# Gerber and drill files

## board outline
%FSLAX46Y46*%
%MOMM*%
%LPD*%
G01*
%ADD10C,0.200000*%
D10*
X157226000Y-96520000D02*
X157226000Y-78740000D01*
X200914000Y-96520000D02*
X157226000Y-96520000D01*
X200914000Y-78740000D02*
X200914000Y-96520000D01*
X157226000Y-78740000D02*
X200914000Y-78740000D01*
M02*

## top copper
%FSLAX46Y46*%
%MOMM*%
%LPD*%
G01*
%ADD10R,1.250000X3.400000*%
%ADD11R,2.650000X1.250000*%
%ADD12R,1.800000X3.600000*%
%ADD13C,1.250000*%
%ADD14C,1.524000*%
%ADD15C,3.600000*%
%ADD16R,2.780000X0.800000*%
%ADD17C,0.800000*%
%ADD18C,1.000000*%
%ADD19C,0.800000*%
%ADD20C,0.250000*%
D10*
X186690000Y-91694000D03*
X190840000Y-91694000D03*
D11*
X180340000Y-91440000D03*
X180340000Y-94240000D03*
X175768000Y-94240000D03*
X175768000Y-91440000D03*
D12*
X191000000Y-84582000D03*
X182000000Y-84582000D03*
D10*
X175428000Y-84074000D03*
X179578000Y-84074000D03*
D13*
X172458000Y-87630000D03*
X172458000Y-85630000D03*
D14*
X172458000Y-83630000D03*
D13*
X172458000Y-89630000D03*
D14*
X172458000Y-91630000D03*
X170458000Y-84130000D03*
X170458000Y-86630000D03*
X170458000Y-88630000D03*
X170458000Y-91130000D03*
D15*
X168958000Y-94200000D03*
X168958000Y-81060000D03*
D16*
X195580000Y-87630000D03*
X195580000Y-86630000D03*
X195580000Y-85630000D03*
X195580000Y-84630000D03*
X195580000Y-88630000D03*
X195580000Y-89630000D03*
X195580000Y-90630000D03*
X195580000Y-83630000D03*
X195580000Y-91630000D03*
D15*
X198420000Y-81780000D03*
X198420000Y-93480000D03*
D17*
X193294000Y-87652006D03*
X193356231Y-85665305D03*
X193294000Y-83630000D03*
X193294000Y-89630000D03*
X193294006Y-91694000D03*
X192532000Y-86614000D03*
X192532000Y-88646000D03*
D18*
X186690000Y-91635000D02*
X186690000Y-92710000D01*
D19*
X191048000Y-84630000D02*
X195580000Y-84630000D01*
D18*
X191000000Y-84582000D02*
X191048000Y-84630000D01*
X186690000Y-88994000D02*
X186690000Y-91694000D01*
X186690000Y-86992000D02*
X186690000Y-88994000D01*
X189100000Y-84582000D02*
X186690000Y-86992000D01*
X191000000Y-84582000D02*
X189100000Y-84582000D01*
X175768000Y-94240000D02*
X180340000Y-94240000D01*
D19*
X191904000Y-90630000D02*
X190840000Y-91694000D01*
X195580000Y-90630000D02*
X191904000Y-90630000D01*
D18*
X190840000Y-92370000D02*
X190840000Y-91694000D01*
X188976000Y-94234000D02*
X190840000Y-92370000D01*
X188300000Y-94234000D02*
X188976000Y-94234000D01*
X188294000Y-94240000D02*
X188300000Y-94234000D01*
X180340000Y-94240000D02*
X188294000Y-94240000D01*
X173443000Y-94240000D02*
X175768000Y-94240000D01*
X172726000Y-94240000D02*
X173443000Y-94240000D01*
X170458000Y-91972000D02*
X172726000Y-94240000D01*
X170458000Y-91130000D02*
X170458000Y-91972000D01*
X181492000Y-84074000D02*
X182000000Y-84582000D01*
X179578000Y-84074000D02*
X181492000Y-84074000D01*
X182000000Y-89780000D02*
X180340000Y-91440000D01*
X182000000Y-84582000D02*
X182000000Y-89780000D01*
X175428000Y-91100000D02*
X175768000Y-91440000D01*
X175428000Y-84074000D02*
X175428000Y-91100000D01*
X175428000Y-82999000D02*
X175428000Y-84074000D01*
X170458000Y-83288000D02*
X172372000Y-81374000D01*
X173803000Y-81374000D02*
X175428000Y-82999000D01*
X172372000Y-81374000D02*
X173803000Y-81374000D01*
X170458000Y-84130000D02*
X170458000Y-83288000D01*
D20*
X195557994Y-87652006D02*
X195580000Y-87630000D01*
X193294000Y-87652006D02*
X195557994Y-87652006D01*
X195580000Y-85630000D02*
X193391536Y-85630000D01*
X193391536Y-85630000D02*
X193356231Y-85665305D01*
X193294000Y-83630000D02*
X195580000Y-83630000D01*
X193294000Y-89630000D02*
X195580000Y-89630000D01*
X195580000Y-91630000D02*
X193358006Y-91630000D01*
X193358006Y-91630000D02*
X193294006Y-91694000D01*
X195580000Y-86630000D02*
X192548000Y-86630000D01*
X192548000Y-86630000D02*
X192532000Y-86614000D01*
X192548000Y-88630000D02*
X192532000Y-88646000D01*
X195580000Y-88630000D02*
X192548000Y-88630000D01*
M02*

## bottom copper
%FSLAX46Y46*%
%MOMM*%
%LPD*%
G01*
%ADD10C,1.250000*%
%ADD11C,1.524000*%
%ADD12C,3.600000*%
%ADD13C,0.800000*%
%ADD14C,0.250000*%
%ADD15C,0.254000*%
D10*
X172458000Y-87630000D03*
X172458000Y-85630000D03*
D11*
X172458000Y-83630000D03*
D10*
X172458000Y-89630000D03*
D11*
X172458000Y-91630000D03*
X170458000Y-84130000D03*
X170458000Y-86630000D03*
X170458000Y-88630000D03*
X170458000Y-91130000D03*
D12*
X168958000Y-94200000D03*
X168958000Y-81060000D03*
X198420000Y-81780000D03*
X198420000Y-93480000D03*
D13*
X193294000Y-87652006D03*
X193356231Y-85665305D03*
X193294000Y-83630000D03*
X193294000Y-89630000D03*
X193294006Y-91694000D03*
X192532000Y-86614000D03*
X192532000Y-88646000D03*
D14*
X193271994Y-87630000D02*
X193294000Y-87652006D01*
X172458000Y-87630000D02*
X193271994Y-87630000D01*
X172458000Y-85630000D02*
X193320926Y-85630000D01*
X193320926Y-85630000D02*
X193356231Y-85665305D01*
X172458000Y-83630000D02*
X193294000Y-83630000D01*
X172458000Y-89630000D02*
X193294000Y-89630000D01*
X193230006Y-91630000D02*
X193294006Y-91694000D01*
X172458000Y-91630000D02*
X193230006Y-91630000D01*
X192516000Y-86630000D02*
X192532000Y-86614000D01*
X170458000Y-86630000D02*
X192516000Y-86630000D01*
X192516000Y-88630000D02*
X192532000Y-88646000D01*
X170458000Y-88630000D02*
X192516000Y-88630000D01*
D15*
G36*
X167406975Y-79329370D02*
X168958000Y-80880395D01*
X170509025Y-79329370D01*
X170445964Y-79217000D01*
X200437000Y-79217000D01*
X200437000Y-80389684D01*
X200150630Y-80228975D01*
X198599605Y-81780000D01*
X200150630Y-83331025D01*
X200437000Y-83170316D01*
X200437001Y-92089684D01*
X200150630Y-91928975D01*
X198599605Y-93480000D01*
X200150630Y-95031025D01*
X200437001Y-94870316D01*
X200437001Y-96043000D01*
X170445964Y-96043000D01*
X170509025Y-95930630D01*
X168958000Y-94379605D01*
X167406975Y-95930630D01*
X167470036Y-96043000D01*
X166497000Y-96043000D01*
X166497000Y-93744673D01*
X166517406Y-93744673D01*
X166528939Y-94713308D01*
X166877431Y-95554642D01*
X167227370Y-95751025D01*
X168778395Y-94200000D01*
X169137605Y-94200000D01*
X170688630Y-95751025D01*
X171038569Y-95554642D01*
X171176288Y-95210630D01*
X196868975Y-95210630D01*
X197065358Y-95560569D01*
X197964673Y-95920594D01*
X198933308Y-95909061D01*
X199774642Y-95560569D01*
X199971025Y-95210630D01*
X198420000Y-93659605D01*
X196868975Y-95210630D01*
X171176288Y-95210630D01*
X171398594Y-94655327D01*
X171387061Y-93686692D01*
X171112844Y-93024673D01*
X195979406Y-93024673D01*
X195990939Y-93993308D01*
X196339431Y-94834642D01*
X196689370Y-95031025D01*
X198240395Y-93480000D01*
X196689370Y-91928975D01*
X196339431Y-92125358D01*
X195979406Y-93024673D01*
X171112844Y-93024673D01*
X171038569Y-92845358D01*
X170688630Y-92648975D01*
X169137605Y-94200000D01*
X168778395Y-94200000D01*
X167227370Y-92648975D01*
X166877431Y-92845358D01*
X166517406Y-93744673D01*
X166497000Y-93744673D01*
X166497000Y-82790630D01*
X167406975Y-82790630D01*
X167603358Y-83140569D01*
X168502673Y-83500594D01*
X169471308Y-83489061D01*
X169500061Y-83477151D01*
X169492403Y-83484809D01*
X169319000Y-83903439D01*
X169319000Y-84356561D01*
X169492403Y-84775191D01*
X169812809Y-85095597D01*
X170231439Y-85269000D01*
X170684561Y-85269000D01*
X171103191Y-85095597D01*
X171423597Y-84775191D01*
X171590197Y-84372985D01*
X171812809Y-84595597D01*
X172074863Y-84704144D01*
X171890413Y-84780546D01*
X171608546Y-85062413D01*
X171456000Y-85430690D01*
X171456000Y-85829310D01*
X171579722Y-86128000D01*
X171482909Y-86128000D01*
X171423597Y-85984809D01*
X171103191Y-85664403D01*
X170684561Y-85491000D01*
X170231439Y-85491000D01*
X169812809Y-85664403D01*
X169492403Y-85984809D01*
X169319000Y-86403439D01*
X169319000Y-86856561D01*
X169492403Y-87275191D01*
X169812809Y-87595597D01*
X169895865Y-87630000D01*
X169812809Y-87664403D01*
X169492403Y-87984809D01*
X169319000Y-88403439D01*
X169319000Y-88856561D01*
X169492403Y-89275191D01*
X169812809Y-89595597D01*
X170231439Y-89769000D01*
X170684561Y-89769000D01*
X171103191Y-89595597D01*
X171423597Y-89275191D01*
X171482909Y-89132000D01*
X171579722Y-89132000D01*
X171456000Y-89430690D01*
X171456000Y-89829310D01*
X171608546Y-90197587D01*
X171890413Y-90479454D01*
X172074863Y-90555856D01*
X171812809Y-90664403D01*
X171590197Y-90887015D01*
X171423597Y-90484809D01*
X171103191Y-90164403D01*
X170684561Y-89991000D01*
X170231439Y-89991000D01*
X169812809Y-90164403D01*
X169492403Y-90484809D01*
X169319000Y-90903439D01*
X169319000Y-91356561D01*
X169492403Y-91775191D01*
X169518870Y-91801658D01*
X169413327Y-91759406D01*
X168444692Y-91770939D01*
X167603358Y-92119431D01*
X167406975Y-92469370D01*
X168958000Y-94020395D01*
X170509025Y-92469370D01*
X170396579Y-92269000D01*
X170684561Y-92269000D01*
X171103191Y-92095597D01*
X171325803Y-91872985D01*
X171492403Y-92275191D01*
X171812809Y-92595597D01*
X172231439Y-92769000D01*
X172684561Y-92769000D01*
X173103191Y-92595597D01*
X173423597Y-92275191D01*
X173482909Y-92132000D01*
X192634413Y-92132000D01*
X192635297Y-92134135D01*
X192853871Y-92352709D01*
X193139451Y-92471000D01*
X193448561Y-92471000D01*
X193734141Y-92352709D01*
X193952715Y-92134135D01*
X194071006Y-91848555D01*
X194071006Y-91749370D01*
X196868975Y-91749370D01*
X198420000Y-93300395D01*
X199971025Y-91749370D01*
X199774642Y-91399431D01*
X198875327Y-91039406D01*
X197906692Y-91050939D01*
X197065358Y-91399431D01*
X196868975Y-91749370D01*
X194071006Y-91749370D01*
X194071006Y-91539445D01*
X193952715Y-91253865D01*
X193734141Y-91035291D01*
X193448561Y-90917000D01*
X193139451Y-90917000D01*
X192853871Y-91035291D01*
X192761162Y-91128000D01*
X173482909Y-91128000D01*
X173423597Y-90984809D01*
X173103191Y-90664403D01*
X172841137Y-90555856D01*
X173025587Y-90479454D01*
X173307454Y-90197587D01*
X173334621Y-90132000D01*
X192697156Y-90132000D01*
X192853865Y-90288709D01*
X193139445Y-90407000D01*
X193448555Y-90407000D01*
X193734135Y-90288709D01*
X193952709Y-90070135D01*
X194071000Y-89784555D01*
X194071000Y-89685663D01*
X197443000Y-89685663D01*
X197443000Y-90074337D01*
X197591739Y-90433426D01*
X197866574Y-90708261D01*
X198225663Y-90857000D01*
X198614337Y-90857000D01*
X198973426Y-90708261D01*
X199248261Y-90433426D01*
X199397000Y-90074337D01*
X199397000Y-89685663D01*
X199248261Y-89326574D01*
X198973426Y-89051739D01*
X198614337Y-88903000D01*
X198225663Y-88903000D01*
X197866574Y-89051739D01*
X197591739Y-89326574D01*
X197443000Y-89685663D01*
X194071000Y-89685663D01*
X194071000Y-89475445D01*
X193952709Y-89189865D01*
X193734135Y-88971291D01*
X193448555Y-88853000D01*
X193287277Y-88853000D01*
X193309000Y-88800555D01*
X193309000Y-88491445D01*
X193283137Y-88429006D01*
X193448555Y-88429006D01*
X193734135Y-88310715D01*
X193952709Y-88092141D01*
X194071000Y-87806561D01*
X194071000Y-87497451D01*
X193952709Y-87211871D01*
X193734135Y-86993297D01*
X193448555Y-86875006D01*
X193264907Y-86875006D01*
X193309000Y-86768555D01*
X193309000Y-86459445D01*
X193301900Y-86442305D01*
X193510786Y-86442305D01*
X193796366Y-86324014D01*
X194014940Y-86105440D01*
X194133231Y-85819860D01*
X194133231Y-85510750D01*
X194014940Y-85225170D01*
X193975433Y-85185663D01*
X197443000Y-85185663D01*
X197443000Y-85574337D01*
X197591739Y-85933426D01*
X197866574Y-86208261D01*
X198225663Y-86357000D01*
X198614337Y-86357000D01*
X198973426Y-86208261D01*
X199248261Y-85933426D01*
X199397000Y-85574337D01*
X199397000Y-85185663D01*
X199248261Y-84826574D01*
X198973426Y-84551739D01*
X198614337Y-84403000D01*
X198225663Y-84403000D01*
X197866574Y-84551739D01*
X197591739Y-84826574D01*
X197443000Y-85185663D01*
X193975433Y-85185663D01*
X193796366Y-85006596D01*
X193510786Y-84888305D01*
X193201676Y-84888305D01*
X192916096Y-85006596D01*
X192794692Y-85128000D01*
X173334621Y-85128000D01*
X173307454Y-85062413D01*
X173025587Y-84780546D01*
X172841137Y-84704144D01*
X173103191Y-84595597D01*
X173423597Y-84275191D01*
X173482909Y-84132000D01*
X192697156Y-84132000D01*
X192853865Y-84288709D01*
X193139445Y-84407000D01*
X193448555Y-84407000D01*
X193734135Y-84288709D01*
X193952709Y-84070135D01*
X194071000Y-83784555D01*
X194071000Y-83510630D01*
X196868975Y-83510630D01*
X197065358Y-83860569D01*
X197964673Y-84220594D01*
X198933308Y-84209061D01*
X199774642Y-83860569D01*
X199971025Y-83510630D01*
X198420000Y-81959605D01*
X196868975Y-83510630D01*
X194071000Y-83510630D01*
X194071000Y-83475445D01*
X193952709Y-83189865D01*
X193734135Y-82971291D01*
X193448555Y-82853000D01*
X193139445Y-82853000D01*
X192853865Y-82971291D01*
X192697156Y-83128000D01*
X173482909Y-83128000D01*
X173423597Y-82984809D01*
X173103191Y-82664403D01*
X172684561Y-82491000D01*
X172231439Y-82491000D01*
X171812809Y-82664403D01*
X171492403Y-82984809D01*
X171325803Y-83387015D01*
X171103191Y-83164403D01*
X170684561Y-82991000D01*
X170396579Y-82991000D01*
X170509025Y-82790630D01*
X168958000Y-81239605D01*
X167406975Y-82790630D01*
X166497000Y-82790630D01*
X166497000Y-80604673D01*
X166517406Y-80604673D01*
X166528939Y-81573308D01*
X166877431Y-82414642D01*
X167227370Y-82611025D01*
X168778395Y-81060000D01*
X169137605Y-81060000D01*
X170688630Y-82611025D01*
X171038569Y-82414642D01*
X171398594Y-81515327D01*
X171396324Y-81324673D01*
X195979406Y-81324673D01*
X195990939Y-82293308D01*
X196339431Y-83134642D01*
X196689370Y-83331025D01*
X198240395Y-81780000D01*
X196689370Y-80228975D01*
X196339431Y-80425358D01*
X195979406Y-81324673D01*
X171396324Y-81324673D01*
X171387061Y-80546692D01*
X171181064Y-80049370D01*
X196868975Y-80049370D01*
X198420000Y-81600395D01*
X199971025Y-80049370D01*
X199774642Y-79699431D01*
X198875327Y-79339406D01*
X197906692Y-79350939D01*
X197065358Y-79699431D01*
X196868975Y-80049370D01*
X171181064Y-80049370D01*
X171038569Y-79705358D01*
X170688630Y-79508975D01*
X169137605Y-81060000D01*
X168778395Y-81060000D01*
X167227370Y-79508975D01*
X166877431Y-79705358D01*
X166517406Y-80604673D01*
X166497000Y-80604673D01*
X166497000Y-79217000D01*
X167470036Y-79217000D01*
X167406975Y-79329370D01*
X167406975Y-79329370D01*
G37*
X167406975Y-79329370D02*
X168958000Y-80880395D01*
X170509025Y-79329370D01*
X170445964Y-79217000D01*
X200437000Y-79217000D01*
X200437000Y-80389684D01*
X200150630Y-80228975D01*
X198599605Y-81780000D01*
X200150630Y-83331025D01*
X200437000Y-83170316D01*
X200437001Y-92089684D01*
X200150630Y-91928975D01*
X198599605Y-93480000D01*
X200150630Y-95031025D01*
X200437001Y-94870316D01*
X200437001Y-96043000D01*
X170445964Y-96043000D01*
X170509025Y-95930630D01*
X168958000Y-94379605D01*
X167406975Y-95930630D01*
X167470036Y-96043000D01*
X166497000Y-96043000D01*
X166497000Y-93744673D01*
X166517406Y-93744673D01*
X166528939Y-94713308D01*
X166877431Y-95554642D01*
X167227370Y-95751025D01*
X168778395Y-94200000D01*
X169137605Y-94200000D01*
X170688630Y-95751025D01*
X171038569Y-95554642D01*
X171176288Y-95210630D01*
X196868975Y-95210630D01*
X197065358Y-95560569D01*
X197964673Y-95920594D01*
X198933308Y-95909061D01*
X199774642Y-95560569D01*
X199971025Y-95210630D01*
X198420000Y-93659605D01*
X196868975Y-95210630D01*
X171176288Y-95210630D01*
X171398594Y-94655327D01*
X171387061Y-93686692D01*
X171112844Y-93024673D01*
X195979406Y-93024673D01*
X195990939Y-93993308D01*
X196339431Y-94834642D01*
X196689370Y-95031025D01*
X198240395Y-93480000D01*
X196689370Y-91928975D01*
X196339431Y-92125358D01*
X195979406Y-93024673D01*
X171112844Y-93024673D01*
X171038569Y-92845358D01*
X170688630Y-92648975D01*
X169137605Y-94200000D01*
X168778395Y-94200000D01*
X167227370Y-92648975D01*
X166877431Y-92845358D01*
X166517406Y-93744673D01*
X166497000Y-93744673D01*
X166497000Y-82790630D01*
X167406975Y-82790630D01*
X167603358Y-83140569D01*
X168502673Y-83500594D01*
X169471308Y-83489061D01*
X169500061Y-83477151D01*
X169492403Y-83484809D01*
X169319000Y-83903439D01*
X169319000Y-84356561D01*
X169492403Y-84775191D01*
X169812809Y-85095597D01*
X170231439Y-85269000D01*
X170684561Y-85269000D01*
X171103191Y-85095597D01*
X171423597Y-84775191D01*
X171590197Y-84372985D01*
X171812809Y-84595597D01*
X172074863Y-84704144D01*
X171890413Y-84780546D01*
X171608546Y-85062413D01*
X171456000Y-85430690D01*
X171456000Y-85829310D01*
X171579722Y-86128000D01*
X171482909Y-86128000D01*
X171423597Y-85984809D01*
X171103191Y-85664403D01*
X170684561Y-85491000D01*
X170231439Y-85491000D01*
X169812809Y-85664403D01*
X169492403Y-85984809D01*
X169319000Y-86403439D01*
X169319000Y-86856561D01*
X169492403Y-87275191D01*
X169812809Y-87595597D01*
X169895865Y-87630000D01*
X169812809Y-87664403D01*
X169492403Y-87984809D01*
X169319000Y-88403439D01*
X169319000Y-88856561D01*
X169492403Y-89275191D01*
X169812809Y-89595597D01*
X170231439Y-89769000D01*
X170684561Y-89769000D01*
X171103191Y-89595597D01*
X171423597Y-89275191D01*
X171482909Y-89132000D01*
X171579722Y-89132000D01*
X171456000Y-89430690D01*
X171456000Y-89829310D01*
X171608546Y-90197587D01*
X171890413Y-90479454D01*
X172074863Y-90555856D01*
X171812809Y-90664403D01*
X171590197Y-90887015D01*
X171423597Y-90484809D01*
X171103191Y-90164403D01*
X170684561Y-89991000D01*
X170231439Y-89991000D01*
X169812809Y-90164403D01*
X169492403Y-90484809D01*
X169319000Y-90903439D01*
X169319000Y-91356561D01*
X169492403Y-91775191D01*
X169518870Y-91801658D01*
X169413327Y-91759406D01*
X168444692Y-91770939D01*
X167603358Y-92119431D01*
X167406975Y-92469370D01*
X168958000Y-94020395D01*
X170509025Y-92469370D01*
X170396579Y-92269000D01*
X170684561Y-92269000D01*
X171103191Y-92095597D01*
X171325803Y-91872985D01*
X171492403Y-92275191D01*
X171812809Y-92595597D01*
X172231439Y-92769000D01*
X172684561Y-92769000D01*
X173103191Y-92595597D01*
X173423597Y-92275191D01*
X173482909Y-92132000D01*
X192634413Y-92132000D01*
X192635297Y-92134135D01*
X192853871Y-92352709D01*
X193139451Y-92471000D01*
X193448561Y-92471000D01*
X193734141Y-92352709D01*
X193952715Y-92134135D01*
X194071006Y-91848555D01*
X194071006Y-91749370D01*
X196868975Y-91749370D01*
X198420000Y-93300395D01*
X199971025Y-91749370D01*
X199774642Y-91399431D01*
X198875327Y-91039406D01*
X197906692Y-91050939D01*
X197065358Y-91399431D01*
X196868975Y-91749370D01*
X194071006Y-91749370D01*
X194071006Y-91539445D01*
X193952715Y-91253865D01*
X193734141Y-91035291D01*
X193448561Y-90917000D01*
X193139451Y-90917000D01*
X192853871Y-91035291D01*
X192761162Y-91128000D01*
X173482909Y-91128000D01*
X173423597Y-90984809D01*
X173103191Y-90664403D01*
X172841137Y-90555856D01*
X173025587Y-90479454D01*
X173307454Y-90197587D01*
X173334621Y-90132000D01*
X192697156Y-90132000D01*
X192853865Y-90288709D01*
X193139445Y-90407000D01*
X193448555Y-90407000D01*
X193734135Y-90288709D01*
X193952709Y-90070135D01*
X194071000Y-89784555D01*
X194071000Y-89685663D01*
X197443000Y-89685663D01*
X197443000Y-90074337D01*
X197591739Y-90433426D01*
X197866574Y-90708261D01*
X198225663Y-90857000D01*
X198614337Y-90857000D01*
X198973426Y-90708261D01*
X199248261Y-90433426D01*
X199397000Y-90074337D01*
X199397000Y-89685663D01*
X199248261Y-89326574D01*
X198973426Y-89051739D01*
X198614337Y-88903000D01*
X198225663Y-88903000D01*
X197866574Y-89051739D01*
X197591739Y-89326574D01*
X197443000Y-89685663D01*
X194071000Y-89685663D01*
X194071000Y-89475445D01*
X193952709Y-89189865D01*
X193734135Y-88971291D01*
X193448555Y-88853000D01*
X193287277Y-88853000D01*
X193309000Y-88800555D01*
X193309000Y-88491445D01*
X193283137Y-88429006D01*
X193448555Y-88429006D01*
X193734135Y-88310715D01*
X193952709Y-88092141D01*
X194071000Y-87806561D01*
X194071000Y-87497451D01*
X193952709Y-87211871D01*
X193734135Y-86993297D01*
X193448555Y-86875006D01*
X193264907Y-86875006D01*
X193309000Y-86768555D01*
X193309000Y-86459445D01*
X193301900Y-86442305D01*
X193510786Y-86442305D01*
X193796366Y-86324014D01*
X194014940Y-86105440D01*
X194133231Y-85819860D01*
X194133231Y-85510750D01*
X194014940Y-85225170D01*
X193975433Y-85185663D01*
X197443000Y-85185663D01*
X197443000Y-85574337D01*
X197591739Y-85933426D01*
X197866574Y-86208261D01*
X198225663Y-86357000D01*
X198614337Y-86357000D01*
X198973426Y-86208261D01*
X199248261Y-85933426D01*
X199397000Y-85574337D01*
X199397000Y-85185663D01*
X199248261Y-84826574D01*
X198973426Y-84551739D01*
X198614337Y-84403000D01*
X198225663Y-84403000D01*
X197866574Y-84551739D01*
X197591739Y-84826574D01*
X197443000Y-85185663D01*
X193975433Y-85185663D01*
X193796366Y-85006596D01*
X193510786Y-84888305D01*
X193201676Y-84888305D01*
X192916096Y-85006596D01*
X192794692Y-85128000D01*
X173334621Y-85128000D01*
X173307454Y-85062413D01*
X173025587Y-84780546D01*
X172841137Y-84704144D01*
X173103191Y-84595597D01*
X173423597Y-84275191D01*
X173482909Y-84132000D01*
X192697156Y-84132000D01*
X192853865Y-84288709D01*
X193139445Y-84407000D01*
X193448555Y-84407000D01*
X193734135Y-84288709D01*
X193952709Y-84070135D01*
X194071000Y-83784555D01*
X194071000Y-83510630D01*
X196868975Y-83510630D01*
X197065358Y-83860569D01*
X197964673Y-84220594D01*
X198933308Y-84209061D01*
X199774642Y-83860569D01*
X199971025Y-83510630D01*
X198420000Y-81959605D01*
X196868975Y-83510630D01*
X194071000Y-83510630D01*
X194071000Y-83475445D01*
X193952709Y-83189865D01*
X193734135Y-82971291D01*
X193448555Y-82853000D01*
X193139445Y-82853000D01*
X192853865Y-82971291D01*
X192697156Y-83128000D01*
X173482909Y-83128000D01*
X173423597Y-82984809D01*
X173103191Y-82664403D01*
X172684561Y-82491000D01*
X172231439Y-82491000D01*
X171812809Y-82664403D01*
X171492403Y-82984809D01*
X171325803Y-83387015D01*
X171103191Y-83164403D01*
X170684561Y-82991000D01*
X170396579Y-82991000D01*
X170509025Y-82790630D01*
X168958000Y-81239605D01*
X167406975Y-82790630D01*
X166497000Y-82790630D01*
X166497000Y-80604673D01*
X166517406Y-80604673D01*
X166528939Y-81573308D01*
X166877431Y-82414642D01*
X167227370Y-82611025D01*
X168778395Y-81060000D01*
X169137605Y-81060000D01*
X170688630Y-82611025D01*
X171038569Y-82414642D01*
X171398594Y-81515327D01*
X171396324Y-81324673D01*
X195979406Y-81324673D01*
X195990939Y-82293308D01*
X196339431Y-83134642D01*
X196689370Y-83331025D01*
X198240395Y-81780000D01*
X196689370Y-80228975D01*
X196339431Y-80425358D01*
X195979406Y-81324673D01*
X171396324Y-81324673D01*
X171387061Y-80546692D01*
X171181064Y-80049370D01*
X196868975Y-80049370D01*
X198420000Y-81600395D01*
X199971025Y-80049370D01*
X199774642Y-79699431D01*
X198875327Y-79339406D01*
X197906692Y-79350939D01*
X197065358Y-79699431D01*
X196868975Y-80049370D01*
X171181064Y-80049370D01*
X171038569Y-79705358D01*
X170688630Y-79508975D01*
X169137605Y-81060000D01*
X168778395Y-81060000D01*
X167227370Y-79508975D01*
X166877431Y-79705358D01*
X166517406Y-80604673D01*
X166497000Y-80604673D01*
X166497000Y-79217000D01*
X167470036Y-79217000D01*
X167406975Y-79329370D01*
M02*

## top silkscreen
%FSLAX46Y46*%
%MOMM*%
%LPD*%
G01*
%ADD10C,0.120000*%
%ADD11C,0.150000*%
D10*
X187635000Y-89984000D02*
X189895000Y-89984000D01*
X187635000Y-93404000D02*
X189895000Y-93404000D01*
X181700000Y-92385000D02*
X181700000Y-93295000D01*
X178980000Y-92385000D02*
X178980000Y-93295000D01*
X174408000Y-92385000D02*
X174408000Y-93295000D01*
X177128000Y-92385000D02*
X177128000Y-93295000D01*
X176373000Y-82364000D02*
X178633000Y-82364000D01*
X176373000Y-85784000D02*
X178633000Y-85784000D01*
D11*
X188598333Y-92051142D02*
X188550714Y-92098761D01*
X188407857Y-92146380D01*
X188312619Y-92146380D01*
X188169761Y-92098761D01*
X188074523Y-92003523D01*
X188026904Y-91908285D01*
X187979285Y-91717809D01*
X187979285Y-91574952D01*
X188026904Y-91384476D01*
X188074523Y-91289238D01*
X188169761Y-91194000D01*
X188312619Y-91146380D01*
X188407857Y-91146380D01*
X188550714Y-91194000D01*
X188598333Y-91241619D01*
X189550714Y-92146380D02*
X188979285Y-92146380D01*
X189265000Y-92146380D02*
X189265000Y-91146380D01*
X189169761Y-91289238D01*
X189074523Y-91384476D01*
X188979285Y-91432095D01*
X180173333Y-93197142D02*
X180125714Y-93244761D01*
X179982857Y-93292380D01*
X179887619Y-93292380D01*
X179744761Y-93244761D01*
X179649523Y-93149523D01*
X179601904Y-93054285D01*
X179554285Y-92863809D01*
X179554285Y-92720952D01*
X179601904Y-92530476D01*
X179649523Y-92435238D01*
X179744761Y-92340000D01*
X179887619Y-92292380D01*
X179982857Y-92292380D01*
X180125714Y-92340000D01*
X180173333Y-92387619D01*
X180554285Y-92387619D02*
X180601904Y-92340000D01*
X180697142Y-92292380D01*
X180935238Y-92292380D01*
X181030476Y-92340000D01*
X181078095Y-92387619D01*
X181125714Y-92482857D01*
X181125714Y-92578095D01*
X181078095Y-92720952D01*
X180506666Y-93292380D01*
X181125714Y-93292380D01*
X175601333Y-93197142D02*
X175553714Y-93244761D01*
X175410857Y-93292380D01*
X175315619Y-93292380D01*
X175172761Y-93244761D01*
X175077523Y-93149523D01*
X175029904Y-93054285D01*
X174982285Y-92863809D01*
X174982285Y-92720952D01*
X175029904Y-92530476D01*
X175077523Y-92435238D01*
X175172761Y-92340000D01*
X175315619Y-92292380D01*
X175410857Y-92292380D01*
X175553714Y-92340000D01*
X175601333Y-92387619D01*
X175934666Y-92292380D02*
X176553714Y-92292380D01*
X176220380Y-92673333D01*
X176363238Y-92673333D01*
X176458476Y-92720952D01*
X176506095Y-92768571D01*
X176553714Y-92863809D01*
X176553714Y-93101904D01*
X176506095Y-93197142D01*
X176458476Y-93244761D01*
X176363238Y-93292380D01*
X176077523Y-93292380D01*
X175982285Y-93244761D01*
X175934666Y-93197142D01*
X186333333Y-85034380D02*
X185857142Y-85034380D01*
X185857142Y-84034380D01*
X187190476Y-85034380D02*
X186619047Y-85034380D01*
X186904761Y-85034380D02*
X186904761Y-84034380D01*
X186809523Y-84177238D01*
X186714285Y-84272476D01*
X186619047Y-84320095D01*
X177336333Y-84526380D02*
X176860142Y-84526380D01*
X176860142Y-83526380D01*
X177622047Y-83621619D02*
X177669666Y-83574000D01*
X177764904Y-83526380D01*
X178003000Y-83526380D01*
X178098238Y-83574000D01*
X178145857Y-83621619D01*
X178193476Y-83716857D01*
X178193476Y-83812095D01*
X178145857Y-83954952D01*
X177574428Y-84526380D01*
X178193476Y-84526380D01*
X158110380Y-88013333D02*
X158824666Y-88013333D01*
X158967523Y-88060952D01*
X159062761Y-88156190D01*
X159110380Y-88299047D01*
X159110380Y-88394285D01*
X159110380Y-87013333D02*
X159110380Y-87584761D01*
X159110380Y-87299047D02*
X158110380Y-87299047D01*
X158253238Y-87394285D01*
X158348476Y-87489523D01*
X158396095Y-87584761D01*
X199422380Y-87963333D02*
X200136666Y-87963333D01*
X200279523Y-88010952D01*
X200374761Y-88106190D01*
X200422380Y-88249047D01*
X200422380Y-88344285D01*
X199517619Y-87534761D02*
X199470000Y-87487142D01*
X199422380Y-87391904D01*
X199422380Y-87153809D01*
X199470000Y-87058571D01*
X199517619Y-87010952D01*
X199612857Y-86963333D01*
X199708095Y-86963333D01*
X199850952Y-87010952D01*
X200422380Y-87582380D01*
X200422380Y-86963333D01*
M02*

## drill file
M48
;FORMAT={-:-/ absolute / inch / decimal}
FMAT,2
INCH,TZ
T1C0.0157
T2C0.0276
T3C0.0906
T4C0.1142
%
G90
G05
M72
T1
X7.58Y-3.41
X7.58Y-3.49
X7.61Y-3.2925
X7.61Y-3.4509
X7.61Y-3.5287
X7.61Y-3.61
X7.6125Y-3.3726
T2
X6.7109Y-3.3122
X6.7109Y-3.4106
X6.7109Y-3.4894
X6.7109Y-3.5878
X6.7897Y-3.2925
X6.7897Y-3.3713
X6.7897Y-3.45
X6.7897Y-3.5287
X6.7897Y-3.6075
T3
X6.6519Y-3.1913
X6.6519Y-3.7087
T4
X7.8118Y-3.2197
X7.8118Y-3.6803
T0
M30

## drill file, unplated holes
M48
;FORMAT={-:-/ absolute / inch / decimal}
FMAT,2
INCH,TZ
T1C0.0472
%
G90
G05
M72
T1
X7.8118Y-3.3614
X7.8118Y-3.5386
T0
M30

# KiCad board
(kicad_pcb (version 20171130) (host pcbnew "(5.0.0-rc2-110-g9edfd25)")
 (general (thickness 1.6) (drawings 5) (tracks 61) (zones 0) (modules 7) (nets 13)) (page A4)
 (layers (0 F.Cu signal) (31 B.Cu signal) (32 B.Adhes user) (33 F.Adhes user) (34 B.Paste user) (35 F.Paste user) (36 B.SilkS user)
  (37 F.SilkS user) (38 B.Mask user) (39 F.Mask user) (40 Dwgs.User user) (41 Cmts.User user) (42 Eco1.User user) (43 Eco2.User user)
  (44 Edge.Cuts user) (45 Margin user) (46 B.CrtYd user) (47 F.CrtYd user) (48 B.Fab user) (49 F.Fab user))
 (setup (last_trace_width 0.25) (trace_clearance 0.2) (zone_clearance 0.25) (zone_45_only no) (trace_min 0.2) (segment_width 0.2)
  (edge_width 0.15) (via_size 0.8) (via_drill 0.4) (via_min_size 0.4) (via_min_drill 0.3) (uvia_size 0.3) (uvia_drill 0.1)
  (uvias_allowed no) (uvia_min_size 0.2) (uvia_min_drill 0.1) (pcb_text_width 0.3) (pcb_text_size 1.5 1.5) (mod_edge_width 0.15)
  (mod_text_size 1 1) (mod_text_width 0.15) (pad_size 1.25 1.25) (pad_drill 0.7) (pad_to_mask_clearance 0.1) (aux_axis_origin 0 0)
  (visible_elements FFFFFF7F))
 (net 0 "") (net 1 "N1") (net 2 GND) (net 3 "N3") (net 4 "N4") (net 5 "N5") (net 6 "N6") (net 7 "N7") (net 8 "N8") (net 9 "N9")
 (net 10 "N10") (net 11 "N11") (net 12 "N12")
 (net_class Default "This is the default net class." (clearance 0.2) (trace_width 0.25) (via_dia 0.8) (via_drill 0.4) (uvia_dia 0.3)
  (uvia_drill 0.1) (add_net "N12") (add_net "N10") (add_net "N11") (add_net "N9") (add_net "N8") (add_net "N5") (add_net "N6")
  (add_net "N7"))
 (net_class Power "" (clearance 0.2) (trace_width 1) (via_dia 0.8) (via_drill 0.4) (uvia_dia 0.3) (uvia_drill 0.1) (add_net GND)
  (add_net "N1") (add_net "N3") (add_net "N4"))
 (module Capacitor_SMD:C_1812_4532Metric (layer F.Cu) (at 188.765 91.694)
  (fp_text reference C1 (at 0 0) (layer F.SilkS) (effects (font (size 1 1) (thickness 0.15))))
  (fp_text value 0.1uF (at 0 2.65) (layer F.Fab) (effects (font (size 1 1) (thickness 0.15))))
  (fp_line (start -1.13 -1.71) (end 1.13 -1.71) (layer F.SilkS) (width 0.12))
  (fp_line (start -1.13 1.71) (end 1.13 1.71) (layer F.SilkS) (width 0.12))
  (pad 1 smd rect (at -2.075 0) (size 1.25 3.4) (layers F.Cu F.Paste F.Mask) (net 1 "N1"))
  (pad 2 smd rect (at 2.075 0) (size 1.25 3.4) (layers F.Cu F.Paste F.Mask) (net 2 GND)))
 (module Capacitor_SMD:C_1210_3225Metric (layer F.Cu) (at 180.34 92.84 270)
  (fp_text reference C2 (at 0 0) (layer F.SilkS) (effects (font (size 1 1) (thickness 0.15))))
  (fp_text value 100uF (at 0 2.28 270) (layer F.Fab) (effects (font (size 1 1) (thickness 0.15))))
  (fp_line (start -0.455 -1.36) (end 0.455 -1.36) (layer F.SilkS) (width 0.12))
  (fp_line (start -0.455 1.36) (end 0.455 1.36) (layer F.SilkS) (width 0.12))
  (pad 1 smd rect (at -1.4 0 270) (size 1.25 2.65) (layers F.Cu F.Paste F.Mask) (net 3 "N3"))
  (pad 2 smd rect (at 1.4 0 270) (size 1.25 2.65) (layers F.Cu F.Paste F.Mask) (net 2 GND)))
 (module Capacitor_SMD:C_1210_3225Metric (layer F.Cu) (at 175.768 92.84 270)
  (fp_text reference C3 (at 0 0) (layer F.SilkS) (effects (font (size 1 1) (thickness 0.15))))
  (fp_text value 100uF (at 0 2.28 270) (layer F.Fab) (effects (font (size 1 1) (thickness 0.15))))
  (fp_line (start -0.455 1.36) (end 0.455 1.36) (layer F.SilkS) (width 0.12))
  (fp_line (start -0.455 -1.36) (end 0.455 -1.36) (layer F.SilkS) (width 0.12))
  (pad 2 smd rect (at 1.4 0 270) (size 1.25 2.65) (layers F.Cu F.Paste F.Mask) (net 2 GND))
  (pad 1 smd rect (at -1.4 0 270) (size 1.25 2.65) (layers F.Cu F.Paste F.Mask) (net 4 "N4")))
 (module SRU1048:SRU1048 (layer F.Cu) (at 186.5 84.582)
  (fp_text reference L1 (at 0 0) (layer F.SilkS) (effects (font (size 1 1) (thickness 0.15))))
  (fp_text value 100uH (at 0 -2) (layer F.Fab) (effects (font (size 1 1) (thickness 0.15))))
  (pad 1 smd rect (at 4.5 0) (size 1.8 3.6) (layers F.Cu F.Paste F.Mask) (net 1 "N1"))
  (pad 2 smd rect (at -4.5 0) (size 1.8 3.6) (layers F.Cu F.Paste F.Mask) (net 3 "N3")))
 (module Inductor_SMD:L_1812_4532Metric (layer F.Cu) (at 177.503 84.074)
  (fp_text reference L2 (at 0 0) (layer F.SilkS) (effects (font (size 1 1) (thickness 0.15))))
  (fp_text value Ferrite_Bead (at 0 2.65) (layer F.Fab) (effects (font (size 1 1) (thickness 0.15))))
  (fp_line (start -1.13 -1.71) (end 1.13 -1.71) (layer F.SilkS) (width 0.12))
  (fp_line (start -1.13 1.71) (end 1.13 1.71) (layer F.SilkS) (width 0.12))
  (pad 1 smd rect (at -2.075 0) (size 1.25 3.4) (layers F.Cu F.Paste F.Mask) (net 4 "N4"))
  (pad 2 smd rect (at 2.075 0) (size 1.25 3.4) (layers F.Cu F.Paste F.Mask) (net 3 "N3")))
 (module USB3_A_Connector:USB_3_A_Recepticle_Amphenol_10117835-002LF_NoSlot (layer F.Cu) (at 165.608 87.63 270)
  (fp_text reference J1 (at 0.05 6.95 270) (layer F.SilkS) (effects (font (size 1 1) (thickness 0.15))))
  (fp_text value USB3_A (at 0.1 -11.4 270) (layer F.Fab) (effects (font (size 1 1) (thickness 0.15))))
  (pad 7 thru_hole circle (at 0 -6.85 270) (size 1.25 1.25) (drill 0.7) (layers *.Cu *.Mask) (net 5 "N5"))
  (pad 8 thru_hole circle (at -2 -6.85 270) (size 1.25 1.25) (drill 0.7) (layers *.Cu *.Mask) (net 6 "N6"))
  (pad 9 thru_hole circle (at -4 -6.85 270) (size 1.524 1.524) (drill 0.7) (layers *.Cu *.Mask) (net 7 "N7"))
  (pad 6 thru_hole circle (at 2 -6.85 270) (size 1.25 1.25) (drill 0.7) (layers *.Cu *.Mask) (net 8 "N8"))
  (pad 5 thru_hole circle (at 4 -6.85 270) (size 1.524 1.524) (drill 0.7) (layers *.Cu *.Mask) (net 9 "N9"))
  (pad 1 thru_hole circle (at -3.5 -4.85 270) (size 1.524 1.524) (drill 0.7) (layers *.Cu *.Mask) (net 4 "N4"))
  (pad 2 thru_hole circle (at -1 -4.85 270) (size 1.524 1.524) (drill 0.7) (layers *.Cu *.Mask) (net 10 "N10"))
  (pad 3 thru_hole circle (at 1 -4.85 270) (size 1.524 1.524) (drill 0.7) (layers *.Cu *.Mask) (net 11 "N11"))
  (pad 4 thru_hole circle (at 3.5 -4.85 270) (size 1.524 1.524) (drill 0.7) (layers *.Cu *.Mask) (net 2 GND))
  (pad 10 thru_hole circle (at 6.57 -3.35 270) (size 3.6 3.6) (drill 2.3) (layers *.Cu *.Mask) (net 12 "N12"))
  (pad 10 thru_hole circle (at -6.57 -3.35 270) (size 3.6 3.6) (drill 2.3) (layers *.Cu *.Mask) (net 12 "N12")))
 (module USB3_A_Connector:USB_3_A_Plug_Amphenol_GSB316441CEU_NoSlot (layer F.Cu) (at 200.97 87.63 90)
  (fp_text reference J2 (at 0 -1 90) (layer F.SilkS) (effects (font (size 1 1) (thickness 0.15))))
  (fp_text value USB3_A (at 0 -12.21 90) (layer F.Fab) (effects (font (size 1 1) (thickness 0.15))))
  (pad 7 smd rect (at 0 -5.39 90) (size 0.8 2.78) (layers F.Cu F.Paste F.Mask) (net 5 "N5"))
  (pad 2 smd rect (at 1 -5.39 90) (size 0.8 2.78) (layers F.Cu F.Paste F.Mask) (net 10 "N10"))
  (pad 8 smd rect (at 2 -5.39 90) (size 0.8 2.78) (layers F.Cu F.Paste F.Mask) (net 6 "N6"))
  (pad 1 smd rect (at 3 -5.39 90) (size 0.8 2.78) (layers F.Cu F.Paste F.Mask) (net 1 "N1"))
  (pad 3 smd rect (at -1 -5.39 90) (size 0.8 2.78) (layers F.Cu F.Paste F.Mask) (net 11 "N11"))
  (pad 6 smd rect (at -2 -5.39 90) (size 0.8 2.78) (layers F.Cu F.Paste F.Mask) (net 8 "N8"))
  (pad 4 smd rect (at -3 -5.39 90) (size 0.8 2.78) (layers F.Cu F.Paste F.Mask) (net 2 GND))
  (pad 9 smd rect (at 4 -5.39 90) (size 0.8 2.78) (layers F.Cu F.Paste F.Mask) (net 7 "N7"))
  (pad 5 smd rect (at -4 -5.39 90) (size 0.8 2.78) (layers F.Cu F.Paste F.Mask) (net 9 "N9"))
  (pad 10 thru_hole circle (at 5.85 -2.55 90) (size 3.6 3.6) (drill 2.9) (layers *.Cu *.Mask) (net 12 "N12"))
  (pad 10 thru_hole circle (at -5.85 -2.55 90) (size 3.6 3.6) (drill 2.9) (layers *.Cu *.Mask) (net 12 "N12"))
  (pad "" np_thru_hole circle (at 2.25 -2.55 90) (size 1.2 1.2) (drill 1.2) (layers *.Cu *.Mask))
  (pad "" np_thru_hole circle (at -2.25 -2.55 90) (size 1.2 1.2) (drill 1.2) (layers *.Cu *.Mask)))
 (gr_line (start 157.226 96.52) (end 157.226 78.74) (layer Edge.Cuts) (width 0.2))
 (gr_line (start 200.914 96.52) (end 157.226 96.52) (layer Edge.Cuts) (width 0.2))
 (gr_line (start 200.914 78.74) (end 200.914 96.52) (layer Edge.Cuts) (width 0.2))
 (gr_line (start 157.226 78.74) (end 200.914 78.74) (layer Edge.Cuts) (width 0.2))
 (segment (start 186.69 91.635) (end 186.69 92.71) (width 1) (layer F.Cu) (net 1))
 (segment (start 191.048 84.63) (end 195.58 84.63) (width 0.8) (layer F.Cu) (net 1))
 (segment (start 191 84.582) (end 191.048 84.63) (width 1) (layer F.Cu) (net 1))
 (segment (start 186.69 88.994) (end 186.69 91.694) (width 1) (layer F.Cu) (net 1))
 (segment (start 186.69 86.992) (end 186.69 88.994) (width 1) (layer F.Cu) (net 1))
 (segment (start 189.1 84.582) (end 186.69 86.992) (width 1) (layer F.Cu) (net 1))
 (segment (start 191 84.582) (end 189.1 84.582) (width 1) (layer F.Cu) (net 1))
 (segment (start 175.768 94.24) (end 180.34 94.24) (width 1) (layer F.Cu) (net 2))
 (segment (start 191.904 90.63) (end 190.84 91.694) (width 0.8) (layer F.Cu) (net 2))
 (segment (start 195.58 90.63) (end 191.904 90.63) (width 0.8) (layer F.Cu) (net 2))
 (segment (start 190.84 92.37) (end 190.84 91.694) (width 1) (layer F.Cu) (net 2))
 (segment (start 188.976 94.234) (end 190.84 92.37) (width 1) (layer F.Cu) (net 2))
 (segment (start 188.3 94.234) (end 188.976 94.234) (width 1) (layer F.Cu) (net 2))
 (segment (start 188.294 94.24) (end 188.3 94.234) (width 1) (layer F.Cu) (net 2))
 (segment (start 180.34 94.24) (end 188.294 94.24) (width 1) (layer F.Cu) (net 2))
 (segment (start 173.443 94.24) (end 175.768 94.24) (width 1) (layer F.Cu) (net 2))
 (segment (start 172.726 94.24) (end 173.443 94.24) (width 1) (layer F.Cu) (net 2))
 (segment (start 170.458 91.972) (end 172.726 94.24) (width 1) (layer F.Cu) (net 2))
 (segment (start 170.458 91.13) (end 170.458 91.972) (width 1) (layer F.Cu) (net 2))
 (segment (start 181.492 84.074) (end 182 84.582) (width 1) (layer F.Cu) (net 3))
 (segment (start 179.578 84.074) (end 181.492 84.074) (width 1) (layer F.Cu) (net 3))
 (segment (start 182 89.78) (end 180.34 91.44) (width 1) (layer F.Cu) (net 3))
 (segment (start 182 84.582) (end 182 89.78) (width 1) (layer F.Cu) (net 3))
 (segment (start 175.428 91.1) (end 175.768 91.44) (width 1) (layer F.Cu) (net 4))
 (segment (start 175.428 84.074) (end 175.428 91.1) (width 1) (layer F.Cu) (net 4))
 (segment (start 175.428 82.999) (end 175.428 84.074) (width 1) (layer F.Cu) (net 4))
 (segment (start 170.458 83.288) (end 172.372 81.374) (width 1) (layer F.Cu) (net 4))
 (segment (start 173.803 81.374) (end 175.428 82.999) (width 1) (layer F.Cu) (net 4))
 (segment (start 172.372 81.374) (end 173.803 81.374) (width 1) (layer F.Cu) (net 4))
 (segment (start 170.458 84.13) (end 170.458 83.288) (width 1) (layer F.Cu) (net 4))
 (via (at 193.294 87.652006) (size 0.8) (drill 0.4) (layers F.Cu B.Cu) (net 5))
 (segment (start 193.271994 87.63) (end 193.294 87.652006) (width 0.25) (layer B.Cu) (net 5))
 (segment (start 172.458 87.63) (end 193.271994 87.63) (width 0.25) (layer B.Cu) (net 5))
 (segment (start 195.557994 87.652006) (end 195.58 87.63) (width 0.25) (layer F.Cu) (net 5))
 (segment (start 193.294 87.652006) (end 195.557994 87.652006) (width 0.25) (layer F.Cu) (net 5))
 (segment (start 172.458 85.63) (end 193.320926 85.63) (width 0.25) (layer B.Cu) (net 6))
 (segment (start 195.58 85.63) (end 193.391536 85.63) (width 0.25) (layer F.Cu) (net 6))
 (segment (start 193.391536 85.63) (end 193.356231 85.665305) (width 0.25) (layer F.Cu) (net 6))
 (segment (start 193.320926 85.63) (end 193.356231 85.665305) (width 0.25) (layer B.Cu) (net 6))
 (via (at 193.356231 85.665305) (size 0.8) (drill 0.4) (layers F.Cu B.Cu) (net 6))
 (via (at 193.294 83.63) (size 0.8) (drill 0.4) (layers F.Cu B.Cu) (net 7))
 (segment (start 172.458 83.63) (end 193.294 83.63) (width 0.25) (layer B.Cu) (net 7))
 (segment (start 193.294 83.63) (end 195.58 83.63) (width 0.25) (layer F.Cu) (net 7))
 (via (at 193.294 89.63) (size 0.8) (drill 0.4) (layers F.Cu B.Cu) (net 8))
 (segment (start 172.458 89.63) (end 193.294 89.63) (width 0.25) (layer B.Cu) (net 8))
 (segment (start 193.294 89.63) (end 195.58 89.63) (width 0.25) (layer F.Cu) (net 8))
 (via (at 193.294006 91.694) (size 0.8) (drill 0.4) (layers F.Cu B.Cu) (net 9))
 (segment (start 193.230006 91.63) (end 193.294006 91.694) (width 0.25) (layer B.Cu) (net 9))
 (segment (start 172.458 91.63) (end 193.230006 91.63) (width 0.25) (layer B.Cu) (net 9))
 (segment (start 195.58 91.63) (end 193.358006 91.63) (width 0.25) (layer F.Cu) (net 9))
 (segment (start 193.358006 91.63) (end 193.294006 91.694) (width 0.25) (layer F.Cu) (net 9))
 (segment (start 192.516 86.63) (end 192.532 86.614) (width 0.25) (layer B.Cu) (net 10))
 (via (at 192.532 86.614) (size 0.8) (drill 0.4) (layers F.Cu B.Cu) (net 10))
 (segment (start 170.458 86.63) (end 192.516 86.63) (width 0.25) (layer B.Cu) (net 10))
 (segment (start 195.58 86.63) (end 192.548 86.63) (width 0.25) (layer F.Cu) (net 10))
 (segment (start 192.548 86.63) (end 192.532 86.614) (width 0.25) (layer F.Cu) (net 10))
 (segment (start 192.548 88.63) (end 192.532 88.646) (width 0.25) (layer F.Cu) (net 11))
 (segment (start 192.516 88.63) (end 192.532 88.646) (width 0.25) (layer B.Cu) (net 11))
 (via (at 192.532 88.646) (size 0.8) (drill 0.4) (layers F.Cu B.Cu) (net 11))
 (segment (start 195.58 88.63) (end 192.548 88.63) (width 0.25) (layer F.Cu) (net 11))
 (segment (start 170.458 88.63) (end 192.516 88.63) (width 0.25) (layer B.Cu) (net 11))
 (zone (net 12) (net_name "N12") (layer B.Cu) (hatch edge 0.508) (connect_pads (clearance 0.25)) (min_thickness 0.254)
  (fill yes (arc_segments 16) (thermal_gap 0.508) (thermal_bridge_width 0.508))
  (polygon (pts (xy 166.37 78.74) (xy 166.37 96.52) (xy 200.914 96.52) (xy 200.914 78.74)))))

